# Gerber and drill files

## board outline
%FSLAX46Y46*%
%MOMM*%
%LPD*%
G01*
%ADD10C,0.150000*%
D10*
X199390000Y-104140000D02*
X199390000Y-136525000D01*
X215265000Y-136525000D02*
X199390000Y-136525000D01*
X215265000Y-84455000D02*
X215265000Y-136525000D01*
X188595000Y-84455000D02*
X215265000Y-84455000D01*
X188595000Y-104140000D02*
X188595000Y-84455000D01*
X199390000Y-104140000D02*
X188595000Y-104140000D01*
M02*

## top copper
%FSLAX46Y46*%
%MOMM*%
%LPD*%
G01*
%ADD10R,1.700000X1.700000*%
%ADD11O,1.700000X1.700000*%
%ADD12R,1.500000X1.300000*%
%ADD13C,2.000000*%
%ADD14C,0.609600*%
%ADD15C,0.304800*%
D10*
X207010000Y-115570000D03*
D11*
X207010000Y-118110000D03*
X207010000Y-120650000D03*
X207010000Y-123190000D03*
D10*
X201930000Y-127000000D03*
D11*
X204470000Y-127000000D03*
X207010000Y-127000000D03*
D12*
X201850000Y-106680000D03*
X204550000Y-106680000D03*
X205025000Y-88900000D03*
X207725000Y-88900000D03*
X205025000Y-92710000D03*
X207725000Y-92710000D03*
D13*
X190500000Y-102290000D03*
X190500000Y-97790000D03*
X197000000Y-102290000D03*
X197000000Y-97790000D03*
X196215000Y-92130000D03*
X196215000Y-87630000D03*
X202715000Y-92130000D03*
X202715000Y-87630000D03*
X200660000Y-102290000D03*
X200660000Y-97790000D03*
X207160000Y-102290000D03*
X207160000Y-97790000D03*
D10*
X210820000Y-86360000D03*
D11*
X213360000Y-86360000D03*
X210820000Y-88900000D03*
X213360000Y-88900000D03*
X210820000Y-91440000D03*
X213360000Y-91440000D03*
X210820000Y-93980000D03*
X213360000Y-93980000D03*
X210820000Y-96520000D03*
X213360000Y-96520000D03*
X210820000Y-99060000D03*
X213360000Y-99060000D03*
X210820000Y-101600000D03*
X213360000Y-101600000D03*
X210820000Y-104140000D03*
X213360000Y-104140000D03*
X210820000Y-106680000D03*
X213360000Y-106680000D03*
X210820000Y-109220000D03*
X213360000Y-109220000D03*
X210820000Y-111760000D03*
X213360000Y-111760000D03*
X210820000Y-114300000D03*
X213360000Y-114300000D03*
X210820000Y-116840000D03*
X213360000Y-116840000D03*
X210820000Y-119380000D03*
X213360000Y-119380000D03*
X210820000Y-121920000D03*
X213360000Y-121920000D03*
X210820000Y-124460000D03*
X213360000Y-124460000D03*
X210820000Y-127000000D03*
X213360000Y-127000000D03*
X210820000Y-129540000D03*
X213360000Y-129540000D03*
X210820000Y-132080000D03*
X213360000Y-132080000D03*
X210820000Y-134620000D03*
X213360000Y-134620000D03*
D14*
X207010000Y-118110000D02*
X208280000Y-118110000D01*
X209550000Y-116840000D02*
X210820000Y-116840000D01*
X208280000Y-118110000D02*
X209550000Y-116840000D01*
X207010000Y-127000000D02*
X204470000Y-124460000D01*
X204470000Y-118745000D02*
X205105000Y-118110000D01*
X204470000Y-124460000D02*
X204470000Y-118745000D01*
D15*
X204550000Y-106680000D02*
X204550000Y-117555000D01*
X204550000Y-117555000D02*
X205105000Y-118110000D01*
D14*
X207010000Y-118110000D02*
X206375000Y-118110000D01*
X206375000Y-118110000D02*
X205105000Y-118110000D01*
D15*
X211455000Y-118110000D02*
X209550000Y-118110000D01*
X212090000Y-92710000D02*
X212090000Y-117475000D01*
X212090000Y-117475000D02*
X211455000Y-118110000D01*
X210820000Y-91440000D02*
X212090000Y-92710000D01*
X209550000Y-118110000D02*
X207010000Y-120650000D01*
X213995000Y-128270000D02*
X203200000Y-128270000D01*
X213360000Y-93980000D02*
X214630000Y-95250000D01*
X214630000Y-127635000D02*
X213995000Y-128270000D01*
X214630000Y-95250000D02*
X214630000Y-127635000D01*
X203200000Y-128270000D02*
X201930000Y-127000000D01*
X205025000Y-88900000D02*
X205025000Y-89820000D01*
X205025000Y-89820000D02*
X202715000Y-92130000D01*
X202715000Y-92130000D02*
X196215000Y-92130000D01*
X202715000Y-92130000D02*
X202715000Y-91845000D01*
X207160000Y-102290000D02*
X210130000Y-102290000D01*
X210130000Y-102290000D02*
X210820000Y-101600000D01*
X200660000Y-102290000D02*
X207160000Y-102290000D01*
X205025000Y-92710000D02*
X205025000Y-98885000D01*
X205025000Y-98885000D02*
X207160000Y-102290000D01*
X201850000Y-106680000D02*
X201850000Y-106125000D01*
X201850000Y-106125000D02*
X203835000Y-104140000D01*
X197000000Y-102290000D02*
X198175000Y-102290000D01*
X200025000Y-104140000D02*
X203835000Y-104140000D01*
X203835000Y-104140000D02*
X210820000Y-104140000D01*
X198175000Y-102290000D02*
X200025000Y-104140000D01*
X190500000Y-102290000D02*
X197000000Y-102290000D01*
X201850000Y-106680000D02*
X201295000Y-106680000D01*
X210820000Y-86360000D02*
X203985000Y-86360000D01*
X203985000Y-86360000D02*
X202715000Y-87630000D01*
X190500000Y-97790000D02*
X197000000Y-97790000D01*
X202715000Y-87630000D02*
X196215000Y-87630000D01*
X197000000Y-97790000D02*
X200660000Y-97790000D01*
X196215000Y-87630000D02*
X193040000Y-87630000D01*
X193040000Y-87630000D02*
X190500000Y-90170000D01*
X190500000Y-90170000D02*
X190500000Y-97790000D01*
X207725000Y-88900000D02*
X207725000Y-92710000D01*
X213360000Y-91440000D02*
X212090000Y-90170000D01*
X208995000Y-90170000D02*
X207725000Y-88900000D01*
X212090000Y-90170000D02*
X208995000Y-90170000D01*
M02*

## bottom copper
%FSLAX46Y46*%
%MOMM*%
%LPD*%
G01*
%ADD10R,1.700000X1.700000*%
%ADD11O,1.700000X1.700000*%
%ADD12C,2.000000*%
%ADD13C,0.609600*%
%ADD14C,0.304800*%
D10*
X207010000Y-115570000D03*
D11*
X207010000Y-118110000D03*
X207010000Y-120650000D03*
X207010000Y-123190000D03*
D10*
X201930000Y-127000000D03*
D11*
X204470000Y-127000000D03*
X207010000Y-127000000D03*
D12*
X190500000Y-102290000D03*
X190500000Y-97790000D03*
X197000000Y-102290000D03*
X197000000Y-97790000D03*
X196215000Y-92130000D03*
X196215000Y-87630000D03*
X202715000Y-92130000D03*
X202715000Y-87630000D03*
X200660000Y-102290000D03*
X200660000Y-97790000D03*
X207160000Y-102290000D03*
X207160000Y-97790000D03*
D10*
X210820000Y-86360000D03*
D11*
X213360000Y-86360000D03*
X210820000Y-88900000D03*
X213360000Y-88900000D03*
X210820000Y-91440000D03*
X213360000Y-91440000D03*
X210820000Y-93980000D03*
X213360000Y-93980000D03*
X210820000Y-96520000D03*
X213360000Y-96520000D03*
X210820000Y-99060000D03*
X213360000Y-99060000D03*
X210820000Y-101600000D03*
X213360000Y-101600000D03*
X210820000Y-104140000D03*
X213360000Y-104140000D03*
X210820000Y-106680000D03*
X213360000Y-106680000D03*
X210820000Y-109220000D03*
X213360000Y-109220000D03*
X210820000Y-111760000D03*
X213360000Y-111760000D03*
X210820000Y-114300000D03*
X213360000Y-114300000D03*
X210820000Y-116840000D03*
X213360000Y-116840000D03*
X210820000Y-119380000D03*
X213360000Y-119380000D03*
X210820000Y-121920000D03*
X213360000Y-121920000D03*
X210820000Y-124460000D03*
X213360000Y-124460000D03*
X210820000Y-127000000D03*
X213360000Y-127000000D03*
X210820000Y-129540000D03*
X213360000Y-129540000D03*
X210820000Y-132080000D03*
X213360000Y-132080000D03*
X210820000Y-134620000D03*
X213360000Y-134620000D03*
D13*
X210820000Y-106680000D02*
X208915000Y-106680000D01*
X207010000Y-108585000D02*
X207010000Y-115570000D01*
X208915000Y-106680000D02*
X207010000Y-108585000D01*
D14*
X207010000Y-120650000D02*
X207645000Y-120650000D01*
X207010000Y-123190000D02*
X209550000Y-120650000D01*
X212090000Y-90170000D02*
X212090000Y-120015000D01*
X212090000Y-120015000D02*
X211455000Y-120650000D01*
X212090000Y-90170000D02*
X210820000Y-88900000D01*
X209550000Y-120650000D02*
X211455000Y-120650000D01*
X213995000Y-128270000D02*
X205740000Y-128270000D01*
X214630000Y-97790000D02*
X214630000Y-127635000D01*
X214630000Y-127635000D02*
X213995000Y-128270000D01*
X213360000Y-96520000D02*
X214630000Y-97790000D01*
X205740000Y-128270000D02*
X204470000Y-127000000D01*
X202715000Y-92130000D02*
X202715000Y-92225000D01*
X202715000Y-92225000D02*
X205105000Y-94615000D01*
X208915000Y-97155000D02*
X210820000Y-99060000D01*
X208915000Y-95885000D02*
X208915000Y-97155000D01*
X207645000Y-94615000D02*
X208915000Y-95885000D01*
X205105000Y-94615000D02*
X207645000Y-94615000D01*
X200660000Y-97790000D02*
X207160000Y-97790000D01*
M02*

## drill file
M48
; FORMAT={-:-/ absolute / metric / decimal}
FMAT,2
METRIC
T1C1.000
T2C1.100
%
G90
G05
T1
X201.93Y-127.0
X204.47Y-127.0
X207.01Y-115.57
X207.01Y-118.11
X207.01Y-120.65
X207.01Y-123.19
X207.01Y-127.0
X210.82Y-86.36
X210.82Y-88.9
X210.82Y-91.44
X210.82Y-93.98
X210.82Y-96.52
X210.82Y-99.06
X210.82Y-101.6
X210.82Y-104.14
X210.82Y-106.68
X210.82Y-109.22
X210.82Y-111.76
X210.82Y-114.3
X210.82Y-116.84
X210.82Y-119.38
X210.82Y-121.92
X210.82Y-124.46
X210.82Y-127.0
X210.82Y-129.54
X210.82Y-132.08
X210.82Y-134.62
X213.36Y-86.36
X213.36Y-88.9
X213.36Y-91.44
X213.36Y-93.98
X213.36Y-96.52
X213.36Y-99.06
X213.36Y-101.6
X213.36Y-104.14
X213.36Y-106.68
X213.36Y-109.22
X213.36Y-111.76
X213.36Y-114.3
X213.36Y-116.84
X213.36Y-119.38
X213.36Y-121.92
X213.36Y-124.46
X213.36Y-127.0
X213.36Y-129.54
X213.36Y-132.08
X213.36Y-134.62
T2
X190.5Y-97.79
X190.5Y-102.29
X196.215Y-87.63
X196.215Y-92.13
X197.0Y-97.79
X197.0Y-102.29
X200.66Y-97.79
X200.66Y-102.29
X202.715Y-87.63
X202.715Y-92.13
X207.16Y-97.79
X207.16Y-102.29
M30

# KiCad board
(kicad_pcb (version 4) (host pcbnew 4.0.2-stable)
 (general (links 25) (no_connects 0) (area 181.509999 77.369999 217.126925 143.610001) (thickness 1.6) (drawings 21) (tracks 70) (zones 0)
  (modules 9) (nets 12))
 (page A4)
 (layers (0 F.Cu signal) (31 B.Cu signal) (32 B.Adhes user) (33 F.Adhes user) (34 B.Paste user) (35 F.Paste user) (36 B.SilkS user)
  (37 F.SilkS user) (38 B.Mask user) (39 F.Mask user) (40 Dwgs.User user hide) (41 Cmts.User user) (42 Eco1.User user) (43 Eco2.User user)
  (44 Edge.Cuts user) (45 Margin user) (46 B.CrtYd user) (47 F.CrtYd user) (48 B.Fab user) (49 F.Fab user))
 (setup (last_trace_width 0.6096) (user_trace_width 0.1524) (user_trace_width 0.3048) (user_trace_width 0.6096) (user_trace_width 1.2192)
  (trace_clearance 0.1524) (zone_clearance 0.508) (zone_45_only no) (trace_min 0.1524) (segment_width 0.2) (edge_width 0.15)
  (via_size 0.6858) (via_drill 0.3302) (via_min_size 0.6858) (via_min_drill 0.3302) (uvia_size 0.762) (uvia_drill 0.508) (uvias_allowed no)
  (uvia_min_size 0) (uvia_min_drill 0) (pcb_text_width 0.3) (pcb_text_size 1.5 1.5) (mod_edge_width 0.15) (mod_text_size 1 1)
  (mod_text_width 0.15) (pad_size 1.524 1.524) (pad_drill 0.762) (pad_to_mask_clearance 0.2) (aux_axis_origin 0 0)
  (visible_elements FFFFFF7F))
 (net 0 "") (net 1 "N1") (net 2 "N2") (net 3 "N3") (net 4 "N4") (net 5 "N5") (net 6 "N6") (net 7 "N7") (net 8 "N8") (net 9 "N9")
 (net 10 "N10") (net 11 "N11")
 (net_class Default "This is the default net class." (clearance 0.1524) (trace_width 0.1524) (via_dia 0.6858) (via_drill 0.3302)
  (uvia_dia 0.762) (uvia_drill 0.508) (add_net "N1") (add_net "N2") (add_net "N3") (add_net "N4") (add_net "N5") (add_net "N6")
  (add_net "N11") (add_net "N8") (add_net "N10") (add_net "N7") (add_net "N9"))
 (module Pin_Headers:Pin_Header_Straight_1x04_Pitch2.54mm (layer F.Cu) (at 207.01 115.57)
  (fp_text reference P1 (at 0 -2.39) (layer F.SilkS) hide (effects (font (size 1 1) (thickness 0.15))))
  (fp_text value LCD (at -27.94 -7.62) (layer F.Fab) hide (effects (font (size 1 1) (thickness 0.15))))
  (pad 1 thru_hole rect (at 0 0) (size 1.7 1.7) (drill 1) (layers *.Cu *.Mask) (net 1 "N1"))
  (pad 2 thru_hole oval (at 0 2.54) (size 1.7 1.7) (drill 1) (layers *.Cu *.Mask) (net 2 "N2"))
  (pad 3 thru_hole oval (at 0 5.08) (size 1.7 1.7) (drill 1) (layers *.Cu *.Mask) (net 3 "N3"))
  (pad 4 thru_hole oval (at 0 7.62) (size 1.7 1.7) (drill 1) (layers *.Cu *.Mask) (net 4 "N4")))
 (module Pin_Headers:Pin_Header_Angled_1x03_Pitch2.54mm (layer B.Cu) (at 201.93 127 270)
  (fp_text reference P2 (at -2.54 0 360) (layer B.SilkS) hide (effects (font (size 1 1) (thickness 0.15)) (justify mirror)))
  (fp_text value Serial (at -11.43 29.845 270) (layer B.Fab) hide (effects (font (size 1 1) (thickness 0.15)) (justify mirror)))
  (pad 1 thru_hole rect (at 0 0 270) (size 1.7 1.7) (drill 1) (layers *.Cu *.Mask) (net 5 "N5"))
  (pad 2 thru_hole oval (at 0 -2.54 270) (size 1.7 1.7) (drill 1) (layers *.Cu *.Mask) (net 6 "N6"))
  (pad 3 thru_hole oval (at 0 -5.08 270) (size 1.7 1.7) (drill 1) (layers *.Cu *.Mask) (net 2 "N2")))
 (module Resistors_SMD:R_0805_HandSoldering (layer F.Cu) (at 203.2 106.68)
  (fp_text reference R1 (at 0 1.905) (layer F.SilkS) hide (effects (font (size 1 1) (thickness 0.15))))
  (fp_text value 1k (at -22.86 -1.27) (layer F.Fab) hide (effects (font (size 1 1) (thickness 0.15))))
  (pad 1 smd rect (at -1.35 0) (size 1.5 1.3) (layers F.Cu F.Paste F.Mask) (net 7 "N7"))
  (pad 2 smd rect (at 1.35 0) (size 1.5 1.3) (layers F.Cu F.Paste F.Mask) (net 2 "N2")))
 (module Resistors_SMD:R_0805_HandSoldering (layer F.Cu) (at 206.375 88.9)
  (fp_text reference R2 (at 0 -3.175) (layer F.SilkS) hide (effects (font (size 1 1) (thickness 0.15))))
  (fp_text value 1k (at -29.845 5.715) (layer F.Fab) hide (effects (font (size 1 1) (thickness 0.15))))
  (pad 1 smd rect (at -1.35 0) (size 1.5 1.3) (layers F.Cu F.Paste F.Mask) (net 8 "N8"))
  (pad 2 smd rect (at 1.35 0) (size 1.5 1.3) (layers F.Cu F.Paste F.Mask) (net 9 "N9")))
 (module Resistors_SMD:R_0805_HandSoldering (layer F.Cu) (at 206.375 92.71)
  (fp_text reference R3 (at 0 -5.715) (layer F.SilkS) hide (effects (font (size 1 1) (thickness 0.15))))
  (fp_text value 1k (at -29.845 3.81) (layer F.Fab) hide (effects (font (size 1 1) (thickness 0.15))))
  (pad 1 smd rect (at -1.35 0) (size 1.5 1.3) (layers F.Cu F.Paste F.Mask) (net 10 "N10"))
  (pad 2 smd rect (at 1.35 0) (size 1.5 1.3) (layers F.Cu F.Paste F.Mask) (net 9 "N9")))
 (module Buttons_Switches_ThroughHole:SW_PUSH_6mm (layer F.Cu) (at 190.5 97.79)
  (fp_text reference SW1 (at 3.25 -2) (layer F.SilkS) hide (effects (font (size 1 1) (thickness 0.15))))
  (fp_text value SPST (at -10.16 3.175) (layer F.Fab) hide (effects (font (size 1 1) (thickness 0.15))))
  (pad 2 thru_hole circle (at 0 4.5 90) (size 2 2) (drill 1.1) (layers *.Cu *.Mask) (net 7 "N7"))
  (pad 1 thru_hole circle (at 0 0 90) (size 2 2) (drill 1.1) (layers *.Cu *.Mask) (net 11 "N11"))
  (pad 2 thru_hole circle (at 6.5 4.5 90) (size 2 2) (drill 1.1) (layers *.Cu *.Mask) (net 7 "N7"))
  (pad 1 thru_hole circle (at 6.5 0 90) (size 2 2) (drill 1.1) (layers *.Cu *.Mask) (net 11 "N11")))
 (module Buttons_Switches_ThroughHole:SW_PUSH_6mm (layer F.Cu) (at 196.215 87.63)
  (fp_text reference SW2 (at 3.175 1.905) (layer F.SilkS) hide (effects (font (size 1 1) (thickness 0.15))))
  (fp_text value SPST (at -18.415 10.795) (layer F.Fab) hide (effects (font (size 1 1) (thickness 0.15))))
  (pad 2 thru_hole circle (at 0 4.5 90) (size 2 2) (drill 1.1) (layers *.Cu *.Mask) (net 8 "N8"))
  (pad 1 thru_hole circle (at 0 0 90) (size 2 2) (drill 1.1) (layers *.Cu *.Mask) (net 11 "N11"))
  (pad 2 thru_hole circle (at 6.5 4.5 90) (size 2 2) (drill 1.1) (layers *.Cu *.Mask) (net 8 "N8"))
  (pad 1 thru_hole circle (at 6.5 0 90) (size 2 2) (drill 1.1) (layers *.Cu *.Mask) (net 11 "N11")))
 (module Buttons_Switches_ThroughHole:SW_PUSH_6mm (layer F.Cu) (at 200.66 97.79)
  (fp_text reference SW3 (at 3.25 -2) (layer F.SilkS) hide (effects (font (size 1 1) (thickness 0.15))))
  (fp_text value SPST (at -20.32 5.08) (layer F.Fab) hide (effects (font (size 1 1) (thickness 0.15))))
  (pad 2 thru_hole circle (at 0 4.5 90) (size 2 2) (drill 1.1) (layers *.Cu *.Mask) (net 10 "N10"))
  (pad 1 thru_hole circle (at 0 0 90) (size 2 2) (drill 1.1) (layers *.Cu *.Mask) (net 11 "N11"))
  (pad 2 thru_hole circle (at 6.5 4.5 90) (size 2 2) (drill 1.1) (layers *.Cu *.Mask) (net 10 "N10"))
  (pad 1 thru_hole circle (at 6.5 0 90) (size 2 2) (drill 1.1) (layers *.Cu *.Mask) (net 11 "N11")))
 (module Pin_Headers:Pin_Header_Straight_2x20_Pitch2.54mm (layer F.Cu) (at 210.82 86.36)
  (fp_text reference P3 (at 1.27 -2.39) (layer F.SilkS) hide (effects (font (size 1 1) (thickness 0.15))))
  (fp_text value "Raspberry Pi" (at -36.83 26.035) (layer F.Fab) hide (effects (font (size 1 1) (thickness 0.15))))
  (pad 1 thru_hole rect (at 0 0) (size 1.7 1.7) (drill 1) (layers *.Cu *.Mask) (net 11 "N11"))
  (pad 2 thru_hole oval (at 2.54 0) (size 1.7 1.7) (drill 1) (layers *.Cu *.Mask))
  (pad 3 thru_hole oval (at 0 2.54) (size 1.7 1.7) (drill 1) (layers *.Cu *.Mask) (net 4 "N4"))
  (pad 4 thru_hole oval (at 2.54 2.54) (size 1.7 1.7) (drill 1) (layers *.Cu *.Mask))
  (pad 5 thru_hole oval (at 0 5.08) (size 1.7 1.7) (drill 1) (layers *.Cu *.Mask) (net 3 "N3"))
  (pad 6 thru_hole oval (at 2.54 5.08) (size 1.7 1.7) (drill 1) (layers *.Cu *.Mask) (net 9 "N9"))
  (pad 7 thru_hole oval (at 0 7.62) (size 1.7 1.7) (drill 1) (layers *.Cu *.Mask))
  (pad 8 thru_hole oval (at 2.54 7.62) (size 1.7 1.7) (drill 1) (layers *.Cu *.Mask) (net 5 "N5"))
  (pad 9 thru_hole oval (at 0 10.16) (size 1.7 1.7) (drill 1) (layers *.Cu *.Mask))
  (pad 10 thru_hole oval (at 2.54 10.16) (size 1.7 1.7) (drill 1) (layers *.Cu *.Mask) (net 6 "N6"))
  (pad 11 thru_hole oval (at 0 12.7) (size 1.7 1.7) (drill 1) (layers *.Cu *.Mask) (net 8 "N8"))
  (pad 12 thru_hole oval (at 2.54 12.7) (size 1.7 1.7) (drill 1) (layers *.Cu *.Mask))
  (pad 13 thru_hole oval (at 0 15.24) (size 1.7 1.7) (drill 1) (layers *.Cu *.Mask) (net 10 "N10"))
  (pad 14 thru_hole oval (at 2.54 15.24) (size 1.7 1.7) (drill 1) (layers *.Cu *.Mask))
  (pad 15 thru_hole oval (at 0 17.78) (size 1.7 1.7) (drill 1) (layers *.Cu *.Mask) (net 7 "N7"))
  (pad 16 thru_hole oval (at 2.54 17.78) (size 1.7 1.7) (drill 1) (layers *.Cu *.Mask))
  (pad 17 thru_hole oval (at 0 20.32) (size 1.7 1.7) (drill 1) (layers *.Cu *.Mask) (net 1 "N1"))
  (pad 18 thru_hole oval (at 2.54 20.32) (size 1.7 1.7) (drill 1) (layers *.Cu *.Mask))
  (pad 19 thru_hole oval (at 0 22.86) (size 1.7 1.7) (drill 1) (layers *.Cu *.Mask))
  (pad 20 thru_hole oval (at 2.54 22.86) (size 1.7 1.7) (drill 1) (layers *.Cu *.Mask))
  (pad 21 thru_hole oval (at 0 25.4) (size 1.7 1.7) (drill 1) (layers *.Cu *.Mask))
  (pad 22 thru_hole oval (at 2.54 25.4) (size 1.7 1.7) (drill 1) (layers *.Cu *.Mask))
  (pad 23 thru_hole oval (at 0 27.94) (size 1.7 1.7) (drill 1) (layers *.Cu *.Mask))
  (pad 24 thru_hole oval (at 2.54 27.94) (size 1.7 1.7) (drill 1) (layers *.Cu *.Mask))
  (pad 25 thru_hole oval (at 0 30.48) (size 1.7 1.7) (drill 1) (layers *.Cu *.Mask) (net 2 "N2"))
  (pad 26 thru_hole oval (at 2.54 30.48) (size 1.7 1.7) (drill 1) (layers *.Cu *.Mask))
  (pad 27 thru_hole oval (at 0 33.02) (size 1.7 1.7) (drill 1) (layers *.Cu *.Mask))
  (pad 28 thru_hole oval (at 2.54 33.02) (size 1.7 1.7) (drill 1) (layers *.Cu *.Mask))
  (pad 29 thru_hole oval (at 0 35.56) (size 1.7 1.7) (drill 1) (layers *.Cu *.Mask))
  (pad 30 thru_hole oval (at 2.54 35.56) (size 1.7 1.7) (drill 1) (layers *.Cu *.Mask))
  (pad 31 thru_hole oval (at 0 38.1) (size 1.7 1.7) (drill 1) (layers *.Cu *.Mask))
  (pad 32 thru_hole oval (at 2.54 38.1) (size 1.7 1.7) (drill 1) (layers *.Cu *.Mask))
  (pad 33 thru_hole oval (at 0 40.64) (size 1.7 1.7) (drill 1) (layers *.Cu *.Mask))
  (pad 34 thru_hole oval (at 2.54 40.64) (size 1.7 1.7) (drill 1) (layers *.Cu *.Mask))
  (pad 35 thru_hole oval (at 0 43.18) (size 1.7 1.7) (drill 1) (layers *.Cu *.Mask))
  (pad 36 thru_hole oval (at 2.54 43.18) (size 1.7 1.7) (drill 1) (layers *.Cu *.Mask))
  (pad 37 thru_hole oval (at 0 45.72) (size 1.7 1.7) (drill 1) (layers *.Cu *.Mask))
  (pad 38 thru_hole oval (at 2.54 45.72) (size 1.7 1.7) (drill 1) (layers *.Cu *.Mask))
  (pad 39 thru_hole oval (at 0 48.26) (size 1.7 1.7) (drill 1) (layers *.Cu *.Mask))
  (pad 40 thru_hole oval (at 2.54 48.26) (size 1.7 1.7) (drill 1) (layers *.Cu *.Mask)))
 (gr_line (start 199.39 104.14) (end 199.39 136.525) (angle 90) (layer Edge.Cuts) (width 0.15))
 (gr_line (start 215.265 136.525) (end 199.39 136.525) (angle 90) (layer Edge.Cuts) (width 0.15))
 (gr_line (start 215.265 84.455) (end 215.265 136.525) (angle 90) (layer Edge.Cuts) (width 0.15))
 (gr_line (start 188.595 84.455) (end 215.265 84.455) (angle 90) (layer Edge.Cuts) (width 0.15))
 (gr_line (start 188.595 104.14) (end 188.595 84.455) (angle 90) (layer Edge.Cuts) (width 0.15))
 (gr_line (start 199.39 104.14) (end 188.595 104.14) (angle 90) (layer Edge.Cuts) (width 0.15))
 (segment (start 210.82 106.68) (end 208.915 106.68) (width 0.6096) (layer B.Cu) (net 1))
 (segment (start 207.01 108.585) (end 207.01 115.57) (width 0.6096) (layer B.Cu) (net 1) (status 20))
 (segment (start 208.915 106.68) (end 207.01 108.585) (width 0.6096) (layer B.Cu) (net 1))
 (segment (start 207.01 118.11) (end 208.28 118.11) (width 0.6096) (layer F.Cu) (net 2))
 (segment (start 209.55 116.84) (end 210.82 116.84) (width 0.6096) (layer F.Cu) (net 2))
 (segment (start 208.28 118.11) (end 209.55 116.84) (width 0.6096) (layer F.Cu) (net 2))
 (segment (start 207.01 127) (end 204.47 124.46) (width 0.6096) (layer F.Cu) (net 2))
 (segment (start 204.47 118.745) (end 205.105 118.11) (width 0.6096) (layer F.Cu) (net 2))
 (segment (start 204.47 124.46) (end 204.47 118.745) (width 0.6096) (layer F.Cu) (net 2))
 (segment (start 204.55 106.68) (end 204.55 117.555) (width 0.3048) (layer F.Cu) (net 2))
 (segment (start 204.55 117.555) (end 205.105 118.11) (width 0.3048) (layer F.Cu) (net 2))
 (segment (start 207.01 118.11) (end 206.375 118.11) (width 0.6096) (layer F.Cu) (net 2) (status 30))
 (segment (start 206.375 118.11) (end 205.105 118.11) (width 0.6096) (layer F.Cu) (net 2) (status 10))
 (segment (start 211.455 118.11) (end 209.55 118.11) (width 0.3048) (layer F.Cu) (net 3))
 (segment (start 212.09 92.71) (end 212.09 117.475) (width 0.3048) (layer F.Cu) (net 3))
 (segment (start 212.09 117.475) (end 211.455 118.11) (width 0.3048) (layer F.Cu) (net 3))
 (segment (start 210.82 91.44) (end 212.09 92.71) (width 0.3048) (layer F.Cu) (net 3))
 (segment (start 209.55 118.11) (end 207.01 120.65) (width 0.3048) (layer F.Cu) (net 3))
 (segment (start 207.01 120.65) (end 207.645 120.65) (width 0.3048) (layer B.Cu) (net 3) (status 30))
 (segment (start 207.01 123.19) (end 209.55 120.65) (width 0.3048) (layer B.Cu) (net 4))
 (segment (start 212.09 90.17) (end 212.09 120.015) (width 0.3048) (layer B.Cu) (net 4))
 (segment (start 212.09 120.015) (end 211.455 120.65) (width 0.3048) (layer B.Cu) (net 4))
 (segment (start 212.09 90.17) (end 210.82 88.9) (width 0.3048) (layer B.Cu) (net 4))
 (segment (start 209.55 120.65) (end 211.455 120.65) (width 0.3048) (layer B.Cu) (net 4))
 (segment (start 213.995 128.27) (end 203.2 128.27) (width 0.3048) (layer F.Cu) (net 5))
 (segment (start 213.36 93.98) (end 214.63 95.25) (width 0.3048) (layer F.Cu) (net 5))
 (segment (start 214.63 127.635) (end 213.995 128.27) (width 0.3048) (layer F.Cu) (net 5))
 (segment (start 214.63 95.25) (end 214.63 127.635) (width 0.3048) (layer F.Cu) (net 5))
 (segment (start 203.2 128.27) (end 201.93 127) (width 0.3048) (layer F.Cu) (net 5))
 (segment (start 213.995 128.27) (end 205.74 128.27) (width 0.3048) (layer B.Cu) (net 6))
 (segment (start 214.63 97.79) (end 214.63 127.635) (width 0.3048) (layer B.Cu) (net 6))
 (segment (start 214.63 127.635) (end 213.995 128.27) (width 0.3048) (layer B.Cu) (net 6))
 (segment (start 213.36 96.52) (end 214.63 97.79) (width 0.3048) (layer B.Cu) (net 6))
 (segment (start 205.74 128.27) (end 204.47 127) (width 0.3048) (layer B.Cu) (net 6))
 (segment (start 205.025 88.9) (end 205.025 89.82) (width 0.3048) (layer F.Cu) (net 8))
 (segment (start 205.025 89.82) (end 202.715 92.13) (width 0.3048) (layer F.Cu) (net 8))
 (segment (start 202.715 92.13) (end 202.715 92.225) (width 0.3048) (layer B.Cu) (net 8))
 (segment (start 202.715 92.225) (end 205.105 94.615) (width 0.3048) (layer B.Cu) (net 8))
 (segment (start 208.915 97.155) (end 210.82 99.06) (width 0.3048) (layer B.Cu) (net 8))
 (segment (start 208.915 95.885) (end 208.915 97.155) (width 0.3048) (layer B.Cu) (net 8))
 (segment (start 207.645 94.615) (end 208.915 95.885) (width 0.3048) (layer B.Cu) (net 8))
 (segment (start 205.105 94.615) (end 207.645 94.615) (width 0.3048) (layer B.Cu) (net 8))
 (segment (start 202.715 92.13) (end 196.215 92.13) (width 0.3048) (layer F.Cu) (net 8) (status 30))
 (segment (start 202.715 92.13) (end 202.715 91.845) (width 0.3048) (layer F.Cu) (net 8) (status 30))
 (segment (start 207.16 102.29) (end 210.13 102.29) (width 0.3048) (layer F.Cu) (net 10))
 (segment (start 210.13 102.29) (end 210.82 101.6) (width 0.3048) (layer F.Cu) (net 10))
 (segment (start 200.66 102.29) (end 207.16 102.29) (width 0.3048) (layer F.Cu) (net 10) (status 30))
 (segment (start 205.025 92.71) (end 205.025 98.885) (width 0.3048) (layer F.Cu) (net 10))
 (segment (start 205.025 98.885) (end 207.16 102.29) (width 0.3048) (layer F.Cu) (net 10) (status 20))
 (segment (start 201.85 106.68) (end 201.85 106.125) (width 0.3048) (layer F.Cu) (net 7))
 (segment (start 201.85 106.125) (end 203.835 104.14) (width 0.3048) (layer F.Cu) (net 7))
 (segment (start 197 102.29) (end 198.175 102.29) (width 0.3048) (layer F.Cu) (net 7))
 (segment (start 200.025 104.14) (end 203.835 104.14) (width 0.3048) (layer F.Cu) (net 7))
 (segment (start 203.835 104.14) (end 210.82 104.14) (width 0.3048) (layer F.Cu) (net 7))
 (segment (start 198.175 102.29) (end 200.025 104.14) (width 0.3048) (layer F.Cu) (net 7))
 (segment (start 190.5 102.29) (end 197 102.29) (width 0.3048) (layer F.Cu) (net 7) (status 30))
 (segment (start 201.85 106.68) (end 201.295 106.68) (width 0.3048) (layer F.Cu) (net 7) (status 30))
 (segment (start 210.82 86.36) (end 203.985 86.36) (width 0.3048) (layer F.Cu) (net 11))
 (segment (start 203.985 86.36) (end 202.715 87.63) (width 0.3048) (layer F.Cu) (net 11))
 (segment (start 200.66 97.79) (end 207.16 97.79) (width 0.3048) (layer B.Cu) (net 11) (status 30))
 (segment (start 190.5 97.79) (end 197 97.79) (width 0.3048) (layer F.Cu) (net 11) (status 30))
 (segment (start 202.715 87.63) (end 196.215 87.63) (width 0.3048) (layer F.Cu) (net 11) (status 30))
 (segment (start 197 97.79) (end 200.66 97.79) (width 0.3048) (layer F.Cu) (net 11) (status 20))
 (segment (start 196.215 87.63) (end 193.04 87.63) (width 0.3048) (layer F.Cu) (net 11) (status 10))
 (segment (start 193.04 87.63) (end 190.5 90.17) (width 0.3048) (layer F.Cu) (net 11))
 (segment (start 190.5 90.17) (end 190.5 97.79) (width 0.3048) (layer F.Cu) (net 11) (status 20))
 (segment (start 207.725 88.9) (end 207.725 92.71) (width 0.3048) (layer F.Cu) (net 9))
 (segment (start 213.36 91.44) (end 212.09 90.17) (width 0.3048) (layer F.Cu) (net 9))
 (segment (start 208.995 90.17) (end 207.725 88.9) (width 0.3048) (layer F.Cu) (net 9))
 (segment (start 212.09 90.17) (end 208.995 90.17) (width 0.3048) (layer F.Cu) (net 9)))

